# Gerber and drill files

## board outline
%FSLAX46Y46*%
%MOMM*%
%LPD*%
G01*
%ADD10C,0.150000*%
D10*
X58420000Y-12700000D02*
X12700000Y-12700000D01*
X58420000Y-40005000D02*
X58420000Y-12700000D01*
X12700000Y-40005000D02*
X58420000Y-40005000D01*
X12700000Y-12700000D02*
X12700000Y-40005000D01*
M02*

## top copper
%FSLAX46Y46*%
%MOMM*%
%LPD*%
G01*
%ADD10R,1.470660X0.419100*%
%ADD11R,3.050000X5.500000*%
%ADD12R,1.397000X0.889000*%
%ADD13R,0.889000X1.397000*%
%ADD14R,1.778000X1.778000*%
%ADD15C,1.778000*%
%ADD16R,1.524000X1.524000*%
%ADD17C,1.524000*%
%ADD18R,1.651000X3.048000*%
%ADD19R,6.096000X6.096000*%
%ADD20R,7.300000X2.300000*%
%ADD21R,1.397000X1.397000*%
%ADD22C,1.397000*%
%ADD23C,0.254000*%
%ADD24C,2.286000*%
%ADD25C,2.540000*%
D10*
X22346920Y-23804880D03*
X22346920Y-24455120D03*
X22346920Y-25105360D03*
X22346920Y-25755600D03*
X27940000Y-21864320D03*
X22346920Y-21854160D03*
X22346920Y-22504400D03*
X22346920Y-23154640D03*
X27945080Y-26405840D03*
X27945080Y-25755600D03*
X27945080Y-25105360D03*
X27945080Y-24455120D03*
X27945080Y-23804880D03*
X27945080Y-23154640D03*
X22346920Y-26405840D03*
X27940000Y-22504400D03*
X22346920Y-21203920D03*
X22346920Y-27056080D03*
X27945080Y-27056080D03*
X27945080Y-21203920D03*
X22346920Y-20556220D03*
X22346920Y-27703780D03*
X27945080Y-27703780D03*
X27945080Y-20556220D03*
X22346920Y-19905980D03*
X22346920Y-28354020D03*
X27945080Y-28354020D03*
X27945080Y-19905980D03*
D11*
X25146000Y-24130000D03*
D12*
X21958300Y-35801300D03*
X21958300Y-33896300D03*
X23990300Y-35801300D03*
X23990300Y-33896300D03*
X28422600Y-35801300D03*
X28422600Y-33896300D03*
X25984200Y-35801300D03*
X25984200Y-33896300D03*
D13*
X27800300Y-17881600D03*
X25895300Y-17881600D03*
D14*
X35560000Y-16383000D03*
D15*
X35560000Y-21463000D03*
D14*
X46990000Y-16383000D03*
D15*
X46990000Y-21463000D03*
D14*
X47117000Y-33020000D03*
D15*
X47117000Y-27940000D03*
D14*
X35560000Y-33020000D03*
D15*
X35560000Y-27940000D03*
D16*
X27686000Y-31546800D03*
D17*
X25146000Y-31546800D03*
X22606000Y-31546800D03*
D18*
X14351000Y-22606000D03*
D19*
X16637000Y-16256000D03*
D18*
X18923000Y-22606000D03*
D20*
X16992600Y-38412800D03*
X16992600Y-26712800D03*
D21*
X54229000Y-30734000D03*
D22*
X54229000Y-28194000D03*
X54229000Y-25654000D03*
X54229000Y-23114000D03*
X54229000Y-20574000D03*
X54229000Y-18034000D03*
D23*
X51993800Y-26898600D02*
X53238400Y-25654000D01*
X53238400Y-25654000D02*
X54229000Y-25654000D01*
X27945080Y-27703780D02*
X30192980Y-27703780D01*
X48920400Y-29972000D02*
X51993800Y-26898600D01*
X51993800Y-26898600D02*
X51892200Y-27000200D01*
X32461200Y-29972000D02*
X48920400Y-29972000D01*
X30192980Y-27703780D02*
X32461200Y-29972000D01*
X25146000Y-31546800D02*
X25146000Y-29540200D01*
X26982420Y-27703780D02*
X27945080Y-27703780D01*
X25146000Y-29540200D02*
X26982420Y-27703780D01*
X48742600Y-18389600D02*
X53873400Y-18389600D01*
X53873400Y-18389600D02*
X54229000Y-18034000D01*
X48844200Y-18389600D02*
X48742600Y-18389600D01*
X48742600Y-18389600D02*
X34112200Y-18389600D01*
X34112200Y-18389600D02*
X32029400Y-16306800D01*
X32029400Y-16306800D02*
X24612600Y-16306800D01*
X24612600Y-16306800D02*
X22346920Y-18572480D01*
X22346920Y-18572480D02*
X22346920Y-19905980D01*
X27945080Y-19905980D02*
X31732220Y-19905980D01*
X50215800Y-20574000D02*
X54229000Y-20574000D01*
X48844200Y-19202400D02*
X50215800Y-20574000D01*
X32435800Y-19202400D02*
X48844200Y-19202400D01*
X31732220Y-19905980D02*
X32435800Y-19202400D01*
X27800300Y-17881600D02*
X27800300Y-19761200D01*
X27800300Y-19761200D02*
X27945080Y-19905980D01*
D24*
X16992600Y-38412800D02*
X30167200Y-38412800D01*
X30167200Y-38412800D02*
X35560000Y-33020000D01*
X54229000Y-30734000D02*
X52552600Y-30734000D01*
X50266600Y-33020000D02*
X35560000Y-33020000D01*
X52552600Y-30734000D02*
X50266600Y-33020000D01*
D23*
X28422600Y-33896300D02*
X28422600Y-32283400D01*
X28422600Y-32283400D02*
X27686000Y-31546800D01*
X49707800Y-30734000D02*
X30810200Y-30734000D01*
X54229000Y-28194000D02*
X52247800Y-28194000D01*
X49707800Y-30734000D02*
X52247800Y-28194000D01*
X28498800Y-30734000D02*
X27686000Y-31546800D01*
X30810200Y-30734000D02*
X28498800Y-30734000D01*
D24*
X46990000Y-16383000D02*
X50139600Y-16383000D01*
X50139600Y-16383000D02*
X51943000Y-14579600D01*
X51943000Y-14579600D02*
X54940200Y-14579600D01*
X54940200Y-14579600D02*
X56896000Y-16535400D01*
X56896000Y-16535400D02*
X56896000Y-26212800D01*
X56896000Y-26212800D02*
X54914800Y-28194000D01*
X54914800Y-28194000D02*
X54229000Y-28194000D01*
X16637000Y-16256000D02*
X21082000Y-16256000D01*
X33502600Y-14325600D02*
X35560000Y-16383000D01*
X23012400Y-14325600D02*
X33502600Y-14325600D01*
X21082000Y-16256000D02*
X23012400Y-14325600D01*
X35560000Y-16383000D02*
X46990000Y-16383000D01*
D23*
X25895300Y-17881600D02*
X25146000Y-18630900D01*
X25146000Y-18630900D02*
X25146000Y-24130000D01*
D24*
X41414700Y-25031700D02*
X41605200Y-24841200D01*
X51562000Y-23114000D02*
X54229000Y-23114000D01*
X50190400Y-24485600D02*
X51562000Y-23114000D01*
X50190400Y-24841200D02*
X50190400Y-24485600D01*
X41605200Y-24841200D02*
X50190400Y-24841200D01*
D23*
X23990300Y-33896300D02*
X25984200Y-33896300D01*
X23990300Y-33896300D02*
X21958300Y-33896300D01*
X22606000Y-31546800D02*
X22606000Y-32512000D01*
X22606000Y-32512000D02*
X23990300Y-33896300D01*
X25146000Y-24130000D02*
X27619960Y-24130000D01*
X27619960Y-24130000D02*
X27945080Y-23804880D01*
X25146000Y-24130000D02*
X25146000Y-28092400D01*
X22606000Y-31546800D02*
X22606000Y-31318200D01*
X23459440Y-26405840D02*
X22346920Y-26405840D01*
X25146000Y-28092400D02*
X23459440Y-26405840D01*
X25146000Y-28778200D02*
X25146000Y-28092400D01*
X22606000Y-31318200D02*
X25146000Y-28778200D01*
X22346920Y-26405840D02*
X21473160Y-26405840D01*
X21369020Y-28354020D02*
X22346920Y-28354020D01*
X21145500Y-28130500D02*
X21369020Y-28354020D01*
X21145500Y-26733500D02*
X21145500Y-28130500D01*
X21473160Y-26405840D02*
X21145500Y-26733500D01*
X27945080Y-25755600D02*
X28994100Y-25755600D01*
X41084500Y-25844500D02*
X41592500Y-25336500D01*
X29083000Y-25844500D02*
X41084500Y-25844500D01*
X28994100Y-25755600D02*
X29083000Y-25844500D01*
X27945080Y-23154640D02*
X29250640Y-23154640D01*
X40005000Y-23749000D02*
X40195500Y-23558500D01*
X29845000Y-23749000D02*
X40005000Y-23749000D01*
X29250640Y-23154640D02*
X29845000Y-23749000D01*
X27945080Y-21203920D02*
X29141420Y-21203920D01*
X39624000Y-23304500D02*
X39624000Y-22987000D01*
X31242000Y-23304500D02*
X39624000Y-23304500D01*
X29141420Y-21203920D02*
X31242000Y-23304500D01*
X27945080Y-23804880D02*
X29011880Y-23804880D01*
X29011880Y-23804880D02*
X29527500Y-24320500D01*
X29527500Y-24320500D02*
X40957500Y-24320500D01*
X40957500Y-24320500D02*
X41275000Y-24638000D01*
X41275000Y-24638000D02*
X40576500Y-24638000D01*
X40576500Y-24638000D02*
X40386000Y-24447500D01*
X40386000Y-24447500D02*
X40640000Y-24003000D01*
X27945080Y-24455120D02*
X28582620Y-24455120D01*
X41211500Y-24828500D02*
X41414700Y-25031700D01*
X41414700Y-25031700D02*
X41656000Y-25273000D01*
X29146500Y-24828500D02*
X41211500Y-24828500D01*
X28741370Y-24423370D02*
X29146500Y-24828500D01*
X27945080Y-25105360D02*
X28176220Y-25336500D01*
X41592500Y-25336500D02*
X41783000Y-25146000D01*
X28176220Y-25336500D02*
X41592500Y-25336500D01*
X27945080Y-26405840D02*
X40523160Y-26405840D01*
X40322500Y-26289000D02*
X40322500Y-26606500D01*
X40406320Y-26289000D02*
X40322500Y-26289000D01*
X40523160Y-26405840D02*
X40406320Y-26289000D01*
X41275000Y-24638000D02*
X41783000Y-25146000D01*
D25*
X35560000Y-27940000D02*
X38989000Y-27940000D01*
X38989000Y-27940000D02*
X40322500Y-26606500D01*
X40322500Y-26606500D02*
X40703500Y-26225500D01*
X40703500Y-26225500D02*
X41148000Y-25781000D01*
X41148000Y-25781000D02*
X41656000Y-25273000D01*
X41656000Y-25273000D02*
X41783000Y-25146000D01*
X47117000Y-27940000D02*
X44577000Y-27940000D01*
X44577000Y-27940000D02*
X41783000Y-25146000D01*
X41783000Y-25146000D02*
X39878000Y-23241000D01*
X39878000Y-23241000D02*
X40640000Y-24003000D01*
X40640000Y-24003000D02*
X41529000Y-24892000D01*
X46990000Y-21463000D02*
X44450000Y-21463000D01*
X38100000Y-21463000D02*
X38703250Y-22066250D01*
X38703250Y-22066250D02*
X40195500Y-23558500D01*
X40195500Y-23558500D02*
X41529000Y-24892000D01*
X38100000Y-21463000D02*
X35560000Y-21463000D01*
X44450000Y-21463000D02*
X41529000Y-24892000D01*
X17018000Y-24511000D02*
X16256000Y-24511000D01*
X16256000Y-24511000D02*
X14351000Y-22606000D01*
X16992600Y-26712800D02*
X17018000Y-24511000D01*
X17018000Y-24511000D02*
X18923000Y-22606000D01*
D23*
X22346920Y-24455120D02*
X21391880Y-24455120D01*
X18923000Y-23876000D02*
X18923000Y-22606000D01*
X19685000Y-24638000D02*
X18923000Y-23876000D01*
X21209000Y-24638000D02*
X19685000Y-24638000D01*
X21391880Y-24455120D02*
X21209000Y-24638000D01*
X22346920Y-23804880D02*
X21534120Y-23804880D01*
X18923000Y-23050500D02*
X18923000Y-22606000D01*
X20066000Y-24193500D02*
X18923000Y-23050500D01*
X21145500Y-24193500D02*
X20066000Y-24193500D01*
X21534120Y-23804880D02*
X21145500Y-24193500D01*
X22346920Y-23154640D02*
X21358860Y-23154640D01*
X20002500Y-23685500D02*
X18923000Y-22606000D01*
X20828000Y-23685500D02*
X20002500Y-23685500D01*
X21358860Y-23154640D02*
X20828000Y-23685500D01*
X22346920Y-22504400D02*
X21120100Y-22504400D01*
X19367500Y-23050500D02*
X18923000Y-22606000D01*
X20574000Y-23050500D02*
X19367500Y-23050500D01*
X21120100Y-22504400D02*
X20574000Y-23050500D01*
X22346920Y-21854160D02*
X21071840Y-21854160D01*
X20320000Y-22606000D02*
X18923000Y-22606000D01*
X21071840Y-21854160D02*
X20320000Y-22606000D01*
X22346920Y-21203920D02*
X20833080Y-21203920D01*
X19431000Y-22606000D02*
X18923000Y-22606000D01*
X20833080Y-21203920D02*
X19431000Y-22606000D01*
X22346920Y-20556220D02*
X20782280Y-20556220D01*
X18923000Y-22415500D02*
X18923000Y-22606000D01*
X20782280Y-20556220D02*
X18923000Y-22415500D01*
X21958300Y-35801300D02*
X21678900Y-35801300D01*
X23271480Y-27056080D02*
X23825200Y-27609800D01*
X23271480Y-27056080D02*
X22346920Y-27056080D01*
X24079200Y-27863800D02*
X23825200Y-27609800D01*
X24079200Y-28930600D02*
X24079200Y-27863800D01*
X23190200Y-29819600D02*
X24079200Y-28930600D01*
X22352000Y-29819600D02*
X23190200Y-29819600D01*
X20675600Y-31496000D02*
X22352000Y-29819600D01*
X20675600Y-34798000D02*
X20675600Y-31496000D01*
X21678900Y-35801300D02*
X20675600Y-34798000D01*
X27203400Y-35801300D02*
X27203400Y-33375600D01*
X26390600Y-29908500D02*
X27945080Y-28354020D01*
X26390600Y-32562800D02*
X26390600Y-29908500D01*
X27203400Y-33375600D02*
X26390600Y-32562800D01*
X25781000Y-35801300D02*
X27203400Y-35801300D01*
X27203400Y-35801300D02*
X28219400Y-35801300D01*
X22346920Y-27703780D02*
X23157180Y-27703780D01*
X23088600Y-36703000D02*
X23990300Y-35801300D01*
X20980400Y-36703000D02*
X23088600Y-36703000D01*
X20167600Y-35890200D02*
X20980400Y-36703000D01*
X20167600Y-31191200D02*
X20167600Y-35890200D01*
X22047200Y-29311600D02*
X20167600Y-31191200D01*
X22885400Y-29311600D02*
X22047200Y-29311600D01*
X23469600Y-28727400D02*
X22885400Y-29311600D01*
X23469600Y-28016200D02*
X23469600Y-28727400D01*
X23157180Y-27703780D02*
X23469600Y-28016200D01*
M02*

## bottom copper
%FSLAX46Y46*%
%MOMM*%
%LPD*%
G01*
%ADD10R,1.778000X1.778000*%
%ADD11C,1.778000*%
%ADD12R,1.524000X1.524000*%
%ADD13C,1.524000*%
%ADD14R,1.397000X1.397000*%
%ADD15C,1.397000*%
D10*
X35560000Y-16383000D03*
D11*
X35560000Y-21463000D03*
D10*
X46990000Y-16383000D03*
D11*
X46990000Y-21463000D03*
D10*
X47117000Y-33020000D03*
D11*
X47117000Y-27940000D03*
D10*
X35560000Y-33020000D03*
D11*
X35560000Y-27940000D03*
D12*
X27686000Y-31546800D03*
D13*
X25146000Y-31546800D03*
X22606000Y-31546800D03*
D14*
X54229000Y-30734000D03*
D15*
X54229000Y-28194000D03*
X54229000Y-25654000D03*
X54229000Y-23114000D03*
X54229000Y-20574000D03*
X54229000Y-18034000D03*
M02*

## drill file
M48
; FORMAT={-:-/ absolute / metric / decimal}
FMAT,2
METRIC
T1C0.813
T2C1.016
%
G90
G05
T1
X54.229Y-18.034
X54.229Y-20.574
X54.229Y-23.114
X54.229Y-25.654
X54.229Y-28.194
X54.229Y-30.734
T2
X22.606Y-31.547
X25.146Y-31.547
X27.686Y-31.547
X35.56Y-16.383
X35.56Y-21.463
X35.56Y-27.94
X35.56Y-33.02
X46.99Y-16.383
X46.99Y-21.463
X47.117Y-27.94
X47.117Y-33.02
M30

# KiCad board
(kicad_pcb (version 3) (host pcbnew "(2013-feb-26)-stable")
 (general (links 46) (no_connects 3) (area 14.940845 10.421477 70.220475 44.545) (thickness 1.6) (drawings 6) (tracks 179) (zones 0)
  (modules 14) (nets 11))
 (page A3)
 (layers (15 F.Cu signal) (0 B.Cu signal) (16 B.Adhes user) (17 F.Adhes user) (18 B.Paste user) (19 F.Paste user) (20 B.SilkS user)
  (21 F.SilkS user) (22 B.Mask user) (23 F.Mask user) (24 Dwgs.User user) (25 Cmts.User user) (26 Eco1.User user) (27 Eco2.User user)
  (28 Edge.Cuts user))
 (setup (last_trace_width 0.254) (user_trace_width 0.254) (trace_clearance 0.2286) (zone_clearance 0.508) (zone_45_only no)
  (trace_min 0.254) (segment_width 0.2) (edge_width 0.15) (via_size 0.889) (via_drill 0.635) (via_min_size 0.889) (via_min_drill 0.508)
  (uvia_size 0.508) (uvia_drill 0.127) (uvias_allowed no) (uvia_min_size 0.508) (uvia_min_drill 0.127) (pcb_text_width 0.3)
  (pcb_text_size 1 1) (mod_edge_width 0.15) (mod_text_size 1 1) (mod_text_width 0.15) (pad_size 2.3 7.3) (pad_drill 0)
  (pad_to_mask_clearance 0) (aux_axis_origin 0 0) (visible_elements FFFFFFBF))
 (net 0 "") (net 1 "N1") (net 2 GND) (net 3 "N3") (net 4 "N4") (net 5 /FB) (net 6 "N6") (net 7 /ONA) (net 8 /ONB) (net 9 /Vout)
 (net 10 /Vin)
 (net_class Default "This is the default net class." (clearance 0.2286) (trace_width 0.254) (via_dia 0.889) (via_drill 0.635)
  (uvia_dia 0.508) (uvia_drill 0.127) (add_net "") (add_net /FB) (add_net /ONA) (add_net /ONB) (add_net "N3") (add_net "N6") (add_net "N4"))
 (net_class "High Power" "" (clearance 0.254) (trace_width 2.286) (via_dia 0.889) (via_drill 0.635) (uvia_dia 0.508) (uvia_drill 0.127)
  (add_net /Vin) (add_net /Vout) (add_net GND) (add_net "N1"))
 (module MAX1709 (layer F.Cu) (at 25.146 24.13 270) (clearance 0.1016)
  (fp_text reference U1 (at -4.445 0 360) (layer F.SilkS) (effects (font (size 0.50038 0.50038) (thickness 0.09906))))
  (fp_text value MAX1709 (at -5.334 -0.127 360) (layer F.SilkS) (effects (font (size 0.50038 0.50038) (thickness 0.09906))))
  (pad 2 smd rect (at -0.32512 2.79908 270) (size 0.4191 1.47066) (layers F.Cu F.Paste F.Mask) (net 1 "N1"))
  (pad 2 smd rect (at 0.32512 2.79908 270) (size 0.4191 1.47066) (layers F.Cu F.Paste F.Mask) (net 1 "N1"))
  (pad 9 smd rect (at 0.97536 2.79908 270) (size 0.4191 1.47066) (layers F.Cu F.Paste F.Mask))
  (pad 10 smd rect (at 1.6256 2.79908 270) (size 0.4191 1.47066) (layers F.Cu F.Paste F.Mask))
  (pad 25 smd rect (at -2.26568 -2.794 270) (size 0.4191 1.47066) (layers F.Cu F.Paste F.Mask))
  (pad 2 smd rect (at -2.27584 2.79908 270) (size 0.4191 1.47066) (layers F.Cu F.Paste F.Mask) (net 1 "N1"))
  (pad 2 smd rect (at -1.6256 2.79908 270) (size 0.4191 1.47066) (layers F.Cu F.Paste F.Mask) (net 1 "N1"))
  (pad 2 smd rect (at -0.97536 2.79908 270) (size 0.4191 1.47066) (layers F.Cu F.Paste F.Mask) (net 1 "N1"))
  (pad 18 smd rect (at 2.27584 -2.79908 270) (size 0.4191 1.47066) (layers F.Cu F.Paste F.Mask) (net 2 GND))
  (pad 18 smd rect (at 1.6256 -2.79908 270) (size 0.4191 1.47066) (layers F.Cu F.Paste F.Mask) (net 2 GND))
  (pad 18 smd rect (at 0.97536 -2.79908 270) (size 0.4191 1.47066) (layers F.Cu F.Paste F.Mask) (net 2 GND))
  (pad 18 smd rect (at 0.32512 -2.79908 270) (size 0.4191 1.47066) (layers F.Cu F.Paste F.Mask) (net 2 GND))
  (pad 18 smd rect (at -0.32512 -2.79908 270) (size 0.4191 1.47066) (layers F.Cu F.Paste F.Mask) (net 2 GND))
  (pad 18 smd rect (at -0.97536 -2.79908 270) (size 0.4191 1.47066) (layers F.Cu F.Paste F.Mask) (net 2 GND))
  (pad 11 smd rect (at 2.27584 2.79908 270) (size 0.4191 1.47066) (layers F.Cu F.Paste F.Mask) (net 2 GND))
  (pad 24 smd rect (at -1.6256 -2.794 270) (size 0.4191 1.47066) (layers F.Cu F.Paste F.Mask))
  (pad 2 smd rect (at -2.92608 2.79908 270) (size 0.4191 1.47066) (layers F.Cu F.Paste F.Mask) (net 1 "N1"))
  (pad 12 smd rect (at 2.92608 2.79908 270) (size 0.4191 1.47066) (layers F.Cu F.Paste F.Mask) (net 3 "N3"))
  (pad 17 smd rect (at 2.92608 -2.79908 270) (size 0.4191 1.47066) (layers F.Cu F.Paste F.Mask))
  (pad 26 smd rect (at -2.92608 -2.79908 270) (size 0.4191 1.47066) (layers F.Cu F.Paste F.Mask) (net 2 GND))
  (pad 2 smd rect (at -3.57378 2.79908 270) (size 0.4191 1.47066) (layers F.Cu F.Paste F.Mask) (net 1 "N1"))
  (pad 13 smd rect (at 3.57378 2.79908 270) (size 0.4191 1.47066) (layers F.Cu F.Paste F.Mask) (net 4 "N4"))
  (pad 16 smd rect (at 3.57378 -2.79908 270) (size 0.4191 1.47066) (layers F.Cu F.Paste F.Mask) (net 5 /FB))
  (pad 27 smd rect (at -3.57378 -2.79908 270) (size 0.4191 1.47066) (layers F.Cu F.Paste F.Mask) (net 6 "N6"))
  (pad 1 smd rect (at -4.22402 2.79908 270) (size 0.4191 1.47066) (layers F.Cu F.Paste F.Mask) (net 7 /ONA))
  (pad 11 smd rect (at 4.22402 2.79908 270) (size 0.4191 1.47066) (layers F.Cu F.Paste F.Mask) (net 2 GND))
  (pad 15 smd rect (at 4.22402 -2.79908 270) (size 0.4191 1.47066) (layers F.Cu F.Paste F.Mask) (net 6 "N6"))
  (pad 28 smd rect (at -4.22402 -2.79908 270) (size 0.4191 1.47066) (layers F.Cu F.Paste F.Mask) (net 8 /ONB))
  (pad 18 smd rect (at 0 0 270) (size 5.5 3.05) (layers F.Cu F.Paste F.Mask) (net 2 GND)))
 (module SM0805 (layer F.Cu) (at 21.9583 34.8488 90)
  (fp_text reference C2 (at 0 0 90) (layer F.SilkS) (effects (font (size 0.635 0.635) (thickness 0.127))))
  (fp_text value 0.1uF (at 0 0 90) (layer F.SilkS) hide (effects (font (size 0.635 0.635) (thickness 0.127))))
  (pad 1 smd rect (at -0.9525 0 90) (size 0.889 1.397) (layers F.Cu F.Paste F.Mask) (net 3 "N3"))
  (pad 2 smd rect (at 0.9525 0 90) (size 0.889 1.397) (layers F.Cu F.Paste F.Mask) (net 2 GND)))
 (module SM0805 (layer F.Cu) (at 23.9903 34.8488 90)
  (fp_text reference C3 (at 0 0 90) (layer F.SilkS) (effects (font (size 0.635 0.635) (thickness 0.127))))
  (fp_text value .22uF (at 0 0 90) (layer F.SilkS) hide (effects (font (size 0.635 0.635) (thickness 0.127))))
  (pad 1 smd rect (at -0.9525 0 90) (size 0.889 1.397) (layers F.Cu F.Paste F.Mask) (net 4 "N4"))
  (pad 2 smd rect (at 0.9525 0 90) (size 0.889 1.397) (layers F.Cu F.Paste F.Mask) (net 2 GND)))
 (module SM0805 (layer F.Cu) (at 28.4226 34.8488 90)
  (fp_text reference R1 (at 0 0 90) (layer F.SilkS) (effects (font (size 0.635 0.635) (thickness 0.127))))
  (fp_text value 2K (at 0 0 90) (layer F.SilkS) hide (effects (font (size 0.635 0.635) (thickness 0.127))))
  (pad 1 smd rect (at -0.9525 0 90) (size 0.889 1.397) (layers F.Cu F.Paste F.Mask) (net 6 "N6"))
  (pad 2 smd rect (at 0.9525 0 90) (size 0.889 1.397) (layers F.Cu F.Paste F.Mask) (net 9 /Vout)))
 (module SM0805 (layer F.Cu) (at 25.9842 34.8488 90)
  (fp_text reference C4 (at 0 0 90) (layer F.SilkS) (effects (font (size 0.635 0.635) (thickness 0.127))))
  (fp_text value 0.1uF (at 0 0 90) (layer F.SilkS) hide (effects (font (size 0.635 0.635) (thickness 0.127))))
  (pad 1 smd rect (at -0.9525 0 90) (size 0.889 1.397) (layers F.Cu F.Paste F.Mask) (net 6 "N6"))
  (pad 2 smd rect (at 0.9525 0 90) (size 0.889 1.397) (layers F.Cu F.Paste F.Mask) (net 2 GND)))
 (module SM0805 (layer F.Cu) (at 26.8478 17.8816 180)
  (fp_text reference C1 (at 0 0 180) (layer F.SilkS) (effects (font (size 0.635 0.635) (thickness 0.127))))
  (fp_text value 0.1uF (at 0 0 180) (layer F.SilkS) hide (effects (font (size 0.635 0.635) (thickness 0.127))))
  (pad 1 smd rect (at -0.9525 0 180) (size 0.889 1.397) (layers F.Cu F.Paste F.Mask) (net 8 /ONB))
  (pad 2 smd rect (at 0.9525 0 180) (size 0.889 1.397) (layers F.Cu F.Paste F.Mask) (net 2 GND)))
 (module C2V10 (layer B.Cu) (at 35.56 18.923 270)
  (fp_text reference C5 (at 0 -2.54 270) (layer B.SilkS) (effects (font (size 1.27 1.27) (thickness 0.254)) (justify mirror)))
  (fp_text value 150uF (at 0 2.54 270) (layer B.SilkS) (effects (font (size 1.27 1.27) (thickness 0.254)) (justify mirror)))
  (pad 1 thru_hole rect (at -2.54 0 270) (size 1.778 1.778) (drill 1.016) (layers *.Cu *.Mask B.SilkS) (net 9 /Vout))
  (pad 2 thru_hole circle (at 2.54 0 270) (size 1.778 1.778) (drill 1.016) (layers *.Cu *.Mask B.SilkS) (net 2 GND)))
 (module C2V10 (layer B.Cu) (at 46.99 18.923 270)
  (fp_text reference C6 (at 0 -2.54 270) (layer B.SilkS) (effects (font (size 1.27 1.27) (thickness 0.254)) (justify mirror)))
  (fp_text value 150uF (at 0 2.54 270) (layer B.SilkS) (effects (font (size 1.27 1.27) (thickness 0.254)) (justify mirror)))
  (pad 1 thru_hole rect (at -2.54 0 270) (size 1.778 1.778) (drill 1.016) (layers *.Cu *.Mask B.SilkS) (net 9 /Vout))
  (pad 2 thru_hole circle (at 2.54 0 270) (size 1.778 1.778) (drill 1.016) (layers *.Cu *.Mask B.SilkS) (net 2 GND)))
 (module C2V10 (layer B.Cu) (at 47.117 30.48 90)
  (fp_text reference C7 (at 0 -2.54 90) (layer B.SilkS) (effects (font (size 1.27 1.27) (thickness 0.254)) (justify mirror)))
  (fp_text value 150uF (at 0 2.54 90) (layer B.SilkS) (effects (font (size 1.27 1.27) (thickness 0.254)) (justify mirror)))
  (pad 1 thru_hole rect (at -2.54 0 90) (size 1.778 1.778) (drill 1.016) (layers *.Cu *.Mask B.SilkS) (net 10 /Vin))
  (pad 2 thru_hole circle (at 2.54 0 90) (size 1.778 1.778) (drill 1.016) (layers *.Cu *.Mask B.SilkS) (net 2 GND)))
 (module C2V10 (layer B.Cu) (at 35.56 30.48 90)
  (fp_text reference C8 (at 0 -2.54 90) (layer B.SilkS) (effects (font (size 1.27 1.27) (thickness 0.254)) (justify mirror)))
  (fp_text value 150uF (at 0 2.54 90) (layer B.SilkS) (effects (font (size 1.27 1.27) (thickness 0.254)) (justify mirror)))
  (pad 1 thru_hole rect (at -2.54 0 90) (size 1.778 1.778) (drill 1.016) (layers *.Cu *.Mask B.SilkS) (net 10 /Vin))
  (pad 2 thru_hole circle (at 2.54 0 90) (size 1.778 1.778) (drill 1.016) (layers *.Cu *.Mask B.SilkS) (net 2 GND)))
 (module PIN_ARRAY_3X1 (layer F.Cu) (at 25.146 31.5468 180)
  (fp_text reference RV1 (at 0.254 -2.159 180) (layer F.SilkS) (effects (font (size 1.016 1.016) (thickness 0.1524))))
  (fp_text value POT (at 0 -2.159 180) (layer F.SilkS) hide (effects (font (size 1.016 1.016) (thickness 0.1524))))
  (pad 1 thru_hole rect (at -2.54 0 180) (size 1.524 1.524) (drill 1.016) (layers *.Cu *.Mask F.SilkS) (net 9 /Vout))
  (pad 2 thru_hole circle (at 0 0 180) (size 1.524 1.524) (drill 1.016) (layers *.Cu *.Mask F.SilkS) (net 5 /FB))
  (pad 3 thru_hole circle (at 2.54 0 180) (size 1.524 1.524) (drill 1.016) (layers *.Cu *.Mask F.SilkS) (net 2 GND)))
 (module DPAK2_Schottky (layer F.Cu) (at 16.637 22.606)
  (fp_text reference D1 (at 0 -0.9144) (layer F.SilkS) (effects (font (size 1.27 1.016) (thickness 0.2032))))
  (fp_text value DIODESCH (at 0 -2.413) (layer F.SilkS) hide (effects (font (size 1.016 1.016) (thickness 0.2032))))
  (pad 1 smd rect (at -2.286 0) (size 1.651 3.048) (layers F.Cu F.Paste F.Mask) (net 1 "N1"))
  (pad 2 smd rect (at 0 -6.35) (size 6.096 6.096) (layers F.Cu F.Paste F.Mask) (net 9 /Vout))
  (pad 1 smd rect (at 2.286 0) (size 1.651 3.048) (layers F.Cu F.Paste F.Mask) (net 1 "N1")))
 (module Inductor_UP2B (layer F.Cu) (at 16.9926 32.5628 90)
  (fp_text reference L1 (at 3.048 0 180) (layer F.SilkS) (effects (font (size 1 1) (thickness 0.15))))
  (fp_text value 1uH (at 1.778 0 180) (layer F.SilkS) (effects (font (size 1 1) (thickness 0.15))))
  (pad 1 smd rect (at -5.85 0 90) (size 2.3 7.3) (layers F.Cu F.Paste F.Mask) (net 10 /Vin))
  (pad 2 smd rect (at 5.85 0 90) (size 2.3 7.3) (layers F.Cu F.Paste F.Mask) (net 1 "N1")))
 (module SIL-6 (layer F.Cu) (at 54.229 24.384 90)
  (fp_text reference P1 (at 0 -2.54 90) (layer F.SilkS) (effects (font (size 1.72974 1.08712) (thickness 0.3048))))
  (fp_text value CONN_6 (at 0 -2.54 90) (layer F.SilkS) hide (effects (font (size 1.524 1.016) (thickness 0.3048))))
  (pad 1 thru_hole rect (at -6.35 0 90) (size 1.397 1.397) (drill 0.8128) (layers *.Cu *.Mask F.SilkS) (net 10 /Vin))
  (pad 2 thru_hole circle (at -3.81 0 90) (size 1.397 1.397) (drill 0.8128) (layers *.Cu *.Mask F.SilkS) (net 9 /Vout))
  (pad 3 thru_hole circle (at -1.27 0 90) (size 1.397 1.397) (drill 0.8128) (layers *.Cu *.Mask F.SilkS) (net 5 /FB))
  (pad 4 thru_hole circle (at 1.27 0 90) (size 1.397 1.397) (drill 0.8128) (layers *.Cu *.Mask F.SilkS) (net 2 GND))
  (pad 5 thru_hole circle (at 3.81 0 90) (size 1.397 1.397) (drill 0.8128) (layers *.Cu *.Mask F.SilkS) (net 8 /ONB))
  (pad 6 thru_hole circle (at 6.35 0 90) (size 1.397 1.397) (drill 0.8128) (layers *.Cu *.Mask F.SilkS) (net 7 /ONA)))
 (gr_line (start 58.42 12.7) (end 12.7 12.7) (angle 90) (layer Edge.Cuts) (width 0.15))
 (gr_line (start 58.42 40.005) (end 58.42 12.7) (angle 90) (layer Edge.Cuts) (width 0.15))
 (gr_line (start 12.7 40.005) (end 58.42 40.005) (angle 90) (layer Edge.Cuts) (width 0.15))
 (gr_line (start 12.7 12.7) (end 12.7 40.005) (angle 90) (layer Edge.Cuts) (width 0.15))
 (segment (start 51.9938 26.8986) (end 53.2384 25.654) (width 0.254) (layer F.Cu) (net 5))
 (segment (start 53.2384 25.654) (end 54.229 25.654) (width 0.254) (layer F.Cu) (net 5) (status 20))
 (segment (start 27.94508 27.70378) (end 30.19298 27.70378) (width 0.254) (layer F.Cu) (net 5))
 (segment (start 48.9204 29.972) (end 51.9938 26.8986) (width 0.254) (layer F.Cu) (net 5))
 (segment (start 51.9938 26.8986) (end 51.8922 27.0002) (width 0.254) (layer F.Cu) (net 5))
 (segment (start 32.4612 29.972) (end 48.9204 29.972) (width 0.254) (layer F.Cu) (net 5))
 (segment (start 30.19298 27.70378) (end 32.4612 29.972) (width 0.254) (layer F.Cu) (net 5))
 (segment (start 25.146 31.5468) (end 25.146 29.5402) (width 0.254) (layer F.Cu) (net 5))
 (segment (start 26.98242 27.70378) (end 27.94508 27.70378) (width 0.254) (layer F.Cu) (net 5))
 (segment (start 25.146 29.5402) (end 26.98242 27.70378) (width 0.254) (layer F.Cu) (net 5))
 (segment (start 48.7426 18.3896) (end 53.8734 18.3896) (width 0.254) (layer F.Cu) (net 7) (status 20))
 (segment (start 53.8734 18.3896) (end 54.229 18.034) (width 0.254) (layer F.Cu) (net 7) (status 30))
 (segment (start 48.8442 18.3896) (end 48.7426 18.3896) (width 0.254) (layer F.Cu) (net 7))
 (segment (start 48.7426 18.3896) (end 34.1122 18.3896) (width 0.254) (layer F.Cu) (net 7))
 (segment (start 34.1122 18.3896) (end 32.0294 16.3068) (width 0.254) (layer F.Cu) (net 7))
 (segment (start 32.0294 16.3068) (end 24.6126 16.3068) (width 0.254) (layer F.Cu) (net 7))
 (segment (start 24.6126 16.3068) (end 22.34692 18.57248) (width 0.254) (layer F.Cu) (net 7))
 (segment (start 22.34692 18.57248) (end 22.34692 19.90598) (width 0.254) (layer F.Cu) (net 7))
 (segment (start 27.94508 19.90598) (end 31.73222 19.90598) (width 0.254) (layer F.Cu) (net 8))
 (segment (start 50.2158 20.574) (end 54.229 20.574) (width 0.254) (layer F.Cu) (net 8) (status 20))
 (segment (start 48.8442 19.2024) (end 50.2158 20.574) (width 0.254) (layer F.Cu) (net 8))
 (segment (start 32.4358 19.2024) (end 48.8442 19.2024) (width 0.254) (layer F.Cu) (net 8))
 (segment (start 31.73222 19.90598) (end 32.4358 19.2024) (width 0.254) (layer F.Cu) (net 8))
 (segment (start 27.8003 17.8816) (end 27.8003 19.7612) (width 0.254) (layer F.Cu) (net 8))
 (segment (start 27.8003 19.7612) (end 27.94508 19.90598) (width 0.254) (layer F.Cu) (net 8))
 (segment (start 16.9926 38.4128) (end 30.1672 38.4128) (width 2.286) (layer F.Cu) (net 10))
 (segment (start 30.1672 38.4128) (end 35.56 33.02) (width 2.286) (layer F.Cu) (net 10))
 (segment (start 54.229 30.734) (end 52.5526 30.734) (width 2.286) (layer F.Cu) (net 10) (status 10))
 (segment (start 50.2666 33.02) (end 35.56 33.02) (width 2.286) (layer F.Cu) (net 10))
 (segment (start 52.5526 30.734) (end 50.2666 33.02) (width 2.286) (layer F.Cu) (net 10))
 (segment (start 28.4226 33.8963) (end 28.4226 32.2834) (width 0.254) (layer F.Cu) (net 9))
 (segment (start 28.4226 32.2834) (end 27.686 31.5468) (width 0.254) (layer F.Cu) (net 9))
 (segment (start 49.7078 30.734) (end 30.8102 30.734) (width 0.254) (layer F.Cu) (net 9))
 (segment (start 54.229 28.194) (end 52.2478 28.194) (width 0.254) (layer F.Cu) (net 9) (status 10))
 (segment (start 49.7078 30.734) (end 52.2478 28.194) (width 0.254) (layer F.Cu) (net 9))
 (segment (start 28.4988 30.734) (end 27.686 31.5468) (width 0.254) (layer F.Cu) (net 9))
 (segment (start 30.8102 30.734) (end 28.4988 30.734) (width 0.254) (layer F.Cu) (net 9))
 (segment (start 46.99 16.383) (end 50.1396 16.383) (width 2.286) (layer F.Cu) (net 9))
 (segment (start 50.1396 16.383) (end 51.943 14.5796) (width 2.286) (layer F.Cu) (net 9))
 (segment (start 51.943 14.5796) (end 54.9402 14.5796) (width 2.286) (layer F.Cu) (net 9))
 (segment (start 54.9402 14.5796) (end 56.896 16.5354) (width 2.286) (layer F.Cu) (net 9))
 (segment (start 56.896 16.5354) (end 56.896 26.2128) (width 2.286) (layer F.Cu) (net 9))
 (segment (start 56.896 26.2128) (end 54.9148 28.194) (width 2.286) (layer F.Cu) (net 9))
 (segment (start 54.9148 28.194) (end 54.229 28.194) (width 2.286) (layer F.Cu) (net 9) (status 20))
 (segment (start 16.637 16.256) (end 21.082 16.256) (width 2.286) (layer F.Cu) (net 9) (status 10))
 (segment (start 33.5026 14.3256) (end 35.56 16.383) (width 2.286) (layer F.Cu) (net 9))
 (segment (start 23.0124 14.3256) (end 33.5026 14.3256) (width 2.286) (layer F.Cu) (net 9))
 (segment (start 21.082 16.256) (end 23.0124 14.3256) (width 2.286) (layer F.Cu) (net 9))
 (segment (start 35.56 16.383) (end 46.99 16.383) (width 2.286) (layer F.Cu) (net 9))
 (segment (start 25.8953 17.8816) (end 25.146 18.6309) (width 0.254) (layer F.Cu) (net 2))
 (segment (start 25.146 18.6309) (end 25.146 24.13) (width 0.254) (layer F.Cu) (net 2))
 (segment (start 41.4147 25.0317) (end 41.6052 24.8412) (width 2.286) (layer F.Cu) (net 2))
 (segment (start 51.562 23.114) (end 54.229 23.114) (width 2.286) (layer F.Cu) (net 2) (status 20))
 (segment (start 50.1904 24.4856) (end 51.562 23.114) (width 2.286) (layer F.Cu) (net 2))
 (segment (start 50.1904 24.8412) (end 50.1904 24.4856) (width 2.286) (layer F.Cu) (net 2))
 (segment (start 41.6052 24.8412) (end 50.1904 24.8412) (width 2.286) (layer F.Cu) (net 2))
 (segment (start 23.9903 33.8963) (end 25.9842 33.8963) (width 0.254) (layer F.Cu) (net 2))
 (segment (start 23.9903 33.8963) (end 21.9583 33.8963) (width 0.254) (layer F.Cu) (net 2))
 (segment (start 22.606 31.5468) (end 22.606 32.512) (width 0.254) (layer F.Cu) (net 2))
 (segment (start 22.606 32.512) (end 23.9903 33.8963) (width 0.254) (layer F.Cu) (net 2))
 (segment (start 25.146 24.13) (end 27.61996 24.13) (width 0.254) (layer F.Cu) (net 2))
 (segment (start 27.61996 24.13) (end 27.94508 23.80488) (width 0.254) (layer F.Cu) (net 2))
 (segment (start 25.146 24.13) (end 25.146 28.0924) (width 0.254) (layer F.Cu) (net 2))
 (segment (start 22.606 31.5468) (end 22.606 31.3182) (width 0.254) (layer F.Cu) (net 2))
 (segment (start 23.45944 26.40584) (end 22.34692 26.40584) (width 0.254) (layer F.Cu) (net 2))
 (segment (start 25.146 28.0924) (end 23.45944 26.40584) (width 0.254) (layer F.Cu) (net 2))
 (segment (start 25.146 28.7782) (end 25.146 28.0924) (width 0.254) (layer F.Cu) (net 2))
 (segment (start 22.606 31.3182) (end 25.146 28.7782) (width 0.254) (layer F.Cu) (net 2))
 (segment (start 22.34692 26.40584) (end 21.47316 26.40584) (width 0.254) (layer F.Cu) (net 2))
 (segment (start 21.36902 28.35402) (end 22.34692 28.35402) (width 0.254) (layer F.Cu) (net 2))
 (segment (start 21.1455 28.1305) (end 21.36902 28.35402) (width 0.254) (layer F.Cu) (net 2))
 (segment (start 21.1455 26.7335) (end 21.1455 28.1305) (width 0.254) (layer F.Cu) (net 2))
 (segment (start 21.47316 26.40584) (end 21.1455 26.7335) (width 0.254) (layer F.Cu) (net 2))
 (segment (start 27.94508 25.7556) (end 28.9941 25.7556) (width 0.254) (layer F.Cu) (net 2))
 (segment (start 41.0845 25.8445) (end 41.5925 25.3365) (width 0.254) (layer F.Cu) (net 2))
 (segment (start 29.083 25.8445) (end 41.0845 25.8445) (width 0.254) (layer F.Cu) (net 2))
 (segment (start 28.9941 25.7556) (end 29.083 25.8445) (width 0.254) (layer F.Cu) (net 2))
 (segment (start 27.94508 23.15464) (end 29.25064 23.15464) (width 0.254) (layer F.Cu) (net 2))
 (segment (start 40.005 23.749) (end 40.1955 23.5585) (width 0.254) (layer F.Cu) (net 2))
 (segment (start 29.845 23.749) (end 40.005 23.749) (width 0.254) (layer F.Cu) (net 2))
 (segment (start 29.25064 23.15464) (end 29.845 23.749) (width 0.254) (layer F.Cu) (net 2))
 (segment (start 27.94508 21.20392) (end 29.14142 21.20392) (width 0.254) (layer F.Cu) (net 2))
 (segment (start 39.624 23.3045) (end 39.624 22.987) (width 0.254) (layer F.Cu) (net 2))
 (segment (start 31.242 23.3045) (end 39.624 23.3045) (width 0.254) (layer F.Cu) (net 2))
 (segment (start 29.14142 21.20392) (end 31.242 23.3045) (width 0.254) (layer F.Cu) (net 2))
 (segment (start 27.94508 23.80488) (end 29.01188 23.80488) (width 0.254) (layer F.Cu) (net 2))
 (segment (start 29.01188 23.80488) (end 29.5275 24.3205) (width 0.254) (layer F.Cu) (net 2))
 (segment (start 29.5275 24.3205) (end 40.9575 24.3205) (width 0.254) (layer F.Cu) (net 2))
 (segment (start 40.9575 24.3205) (end 41.275 24.638) (width 0.254) (layer F.Cu) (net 2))
 (segment (start 41.275 24.638) (end 40.5765 24.638) (width 0.254) (layer F.Cu) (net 2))
 (segment (start 40.5765 24.638) (end 40.386 24.4475) (width 0.254) (layer F.Cu) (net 2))
 (segment (start 40.386 24.4475) (end 40.64 24.003) (width 0.254) (layer F.Cu) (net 2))
 (segment (start 27.94508 24.45512) (end 28.58262 24.45512) (width 0.254) (layer F.Cu) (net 2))
 (segment (start 41.2115 24.8285) (end 41.4147 25.0317) (width 0.254) (layer F.Cu) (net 2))
 (segment (start 41.4147 25.0317) (end 41.656 25.273) (width 0.254) (layer F.Cu) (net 2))
 (segment (start 29.1465 24.8285) (end 41.2115 24.8285) (width 0.254) (layer F.Cu) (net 2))
 (segment (start 28.74137 24.42337) (end 29.1465 24.8285) (width 0.254) (layer F.Cu) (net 2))
 (segment (start 27.94508 25.10536) (end 28.17622 25.3365) (width 0.254) (layer F.Cu) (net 2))
 (segment (start 41.5925 25.3365) (end 41.783 25.146) (width 0.254) (layer F.Cu) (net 2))
 (segment (start 28.17622 25.3365) (end 41.5925 25.3365) (width 0.254) (layer F.Cu) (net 2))
 (segment (start 27.94508 26.40584) (end 40.52316 26.40584) (width 0.254) (layer F.Cu) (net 2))
 (segment (start 40.3225 26.289) (end 40.3225 26.6065) (width 0.254) (layer F.Cu) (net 2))
 (segment (start 40.40632 26.289) (end 40.3225 26.289) (width 0.254) (layer F.Cu) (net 2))
 (segment (start 40.52316 26.40584) (end 40.40632 26.289) (width 0.254) (layer F.Cu) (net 2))
 (segment (start 41.275 24.638) (end 41.783 25.146) (width 0.254) (layer F.Cu) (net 2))
 (segment (start 35.56 27.94) (end 38.989 27.94) (width 2.54) (layer F.Cu) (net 2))
 (segment (start 38.989 27.94) (end 40.3225 26.6065) (width 2.54) (layer F.Cu) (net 2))
 (segment (start 40.3225 26.6065) (end 40.7035 26.2255) (width 2.54) (layer F.Cu) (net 2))
 (segment (start 40.7035 26.2255) (end 41.148 25.781) (width 2.54) (layer F.Cu) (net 2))
 (segment (start 41.148 25.781) (end 41.656 25.273) (width 2.54) (layer F.Cu) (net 2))
 (segment (start 41.656 25.273) (end 41.783 25.146) (width 2.54) (layer F.Cu) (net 2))
 (segment (start 47.117 27.94) (end 44.577 27.94) (width 2.54) (layer F.Cu) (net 2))
 (segment (start 44.577 27.94) (end 41.783 25.146) (width 2.54) (layer F.Cu) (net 2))
 (segment (start 41.783 25.146) (end 39.878 23.241) (width 2.54) (layer F.Cu) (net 2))
 (segment (start 39.878 23.241) (end 40.64 24.003) (width 2.54) (layer F.Cu) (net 2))
 (segment (start 40.64 24.003) (end 41.529 24.892) (width 2.54) (layer F.Cu) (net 2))
 (segment (start 46.99 21.463) (end 44.45 21.463) (width 2.54) (layer F.Cu) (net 2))
 (segment (start 38.1 21.463) (end 38.70325 22.06625) (width 2.54) (layer F.Cu) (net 2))
 (segment (start 38.70325 22.06625) (end 40.1955 23.5585) (width 2.54) (layer F.Cu) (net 2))
 (segment (start 40.1955 23.5585) (end 41.529 24.892) (width 2.54) (layer F.Cu) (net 2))
 (segment (start 38.1 21.463) (end 35.56 21.463) (width 2.54) (layer F.Cu) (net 2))
 (segment (start 44.45 21.463) (end 41.529 24.892) (width 2.54) (layer F.Cu) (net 2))
 (segment (start 17.018 24.511) (end 16.256 24.511) (width 2.54) (layer F.Cu) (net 1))
 (segment (start 16.256 24.511) (end 14.351 22.606) (width 2.54) (layer F.Cu) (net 1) (status 20))
 (segment (start 16.9926 26.7128) (end 17.018 24.511) (width 2.54) (layer F.Cu) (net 1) (status 10))
 (segment (start 17.018 24.511) (end 18.923 22.606) (width 2.54) (layer F.Cu) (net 1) (status 20))
 (segment (start 22.34692 24.45512) (end 21.39188 24.45512) (width 0.254) (layer F.Cu) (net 1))
 (segment (start 18.923 23.876) (end 18.923 22.606) (width 0.254) (layer F.Cu) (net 1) (status 30))
 (segment (start 19.685 24.638) (end 18.923 23.876) (width 0.254) (layer F.Cu) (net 1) (status 20))
 (segment (start 21.209 24.638) (end 19.685 24.638) (width 0.254) (layer F.Cu) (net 1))
 (segment (start 21.39188 24.45512) (end 21.209 24.638) (width 0.254) (layer F.Cu) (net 1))
 (segment (start 22.34692 23.80488) (end 21.53412 23.80488) (width 0.254) (layer F.Cu) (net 1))
 (segment (start 18.923 23.0505) (end 18.923 22.606) (width 0.254) (layer F.Cu) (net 1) (status 30))
 (segment (start 20.066 24.1935) (end 18.923 23.0505) (width 0.254) (layer F.Cu) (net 1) (status 20))
 (segment (start 21.1455 24.1935) (end 20.066 24.1935) (width 0.254) (layer F.Cu) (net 1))
 (segment (start 21.53412 23.80488) (end 21.1455 24.1935) (width 0.254) (layer F.Cu) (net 1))
 (segment (start 22.34692 23.15464) (end 21.35886 23.15464) (width 0.254) (layer F.Cu) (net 1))
 (segment (start 20.0025 23.6855) (end 18.923 22.606) (width 0.254) (layer F.Cu) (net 1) (status 20))
 (segment (start 20.828 23.6855) (end 20.0025 23.6855) (width 0.254) (layer F.Cu) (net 1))
 (segment (start 21.35886 23.15464) (end 20.828 23.6855) (width 0.254) (layer F.Cu) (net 1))
 (segment (start 22.34692 22.5044) (end 21.1201 22.5044) (width 0.254) (layer F.Cu) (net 1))
 (segment (start 19.3675 23.0505) (end 18.923 22.606) (width 0.254) (layer F.Cu) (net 1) (status 30))
 (segment (start 20.574 23.0505) (end 19.3675 23.0505) (width 0.254) (layer F.Cu) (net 1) (status 20))
 (segment (start 21.1201 22.5044) (end 20.574 23.0505) (width 0.254) (layer F.Cu) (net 1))
 (segment (start 22.34692 21.85416) (end 21.07184 21.85416) (width 0.254) (layer F.Cu) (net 1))
 (segment (start 20.32 22.606) (end 18.923 22.606) (width 0.254) (layer F.Cu) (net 1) (status 20))
 (segment (start 21.07184 21.85416) (end 20.32 22.606) (width 0.254) (layer F.Cu) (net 1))
 (segment (start 22.34692 21.20392) (end 20.83308 21.20392) (width 0.254) (layer F.Cu) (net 1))
 (segment (start 19.431 22.606) (end 18.923 22.606) (width 0.254) (layer F.Cu) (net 1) (status 30))
 (segment (start 20.83308 21.20392) (end 19.431 22.606) (width 0.254) (layer F.Cu) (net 1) (status 20))
 (segment (start 22.34692 20.55622) (end 20.78228 20.55622) (width 0.254) (layer F.Cu) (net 1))
 (segment (start 18.923 22.4155) (end 18.923 22.606) (width 0.254) (layer F.Cu) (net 1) (status 30))
 (segment (start 20.78228 20.55622) (end 18.923 22.4155) (width 0.254) (layer F.Cu) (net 1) (status 20))
 (segment (start 21.9583 35.8013) (end 21.6789 35.8013) (width 0.254) (layer F.Cu) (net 3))
 (segment (start 23.27148 27.05608) (end 23.8252 27.6098) (width 0.254) (layer F.Cu) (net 3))
 (segment (start 23.27148 27.05608) (end 22.34692 27.05608) (width 0.254) (layer F.Cu) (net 3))
 (segment (start 24.0792 27.8638) (end 23.8252 27.6098) (width 0.254) (layer F.Cu) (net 3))
 (segment (start 24.0792 28.9306) (end 24.0792 27.8638) (width 0.254) (layer F.Cu) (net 3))
 (segment (start 23.1902 29.8196) (end 24.0792 28.9306) (width 0.254) (layer F.Cu) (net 3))
 (segment (start 22.352 29.8196) (end 23.1902 29.8196) (width 0.254) (layer F.Cu) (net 3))
 (segment (start 20.6756 31.496) (end 22.352 29.8196) (width 0.254) (layer F.Cu) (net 3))
 (segment (start 20.6756 34.798) (end 20.6756 31.496) (width 0.254) (layer F.Cu) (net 3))
 (segment (start 21.6789 35.8013) (end 20.6756 34.798) (width 0.254) (layer F.Cu) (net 3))
 (segment (start 27.2034 35.8013) (end 27.2034 33.3756) (width 0.254) (layer F.Cu) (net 6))
 (segment (start 26.3906 29.9085) (end 27.94508 28.35402) (width 0.254) (layer F.Cu) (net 6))
 (segment (start 26.3906 32.5628) (end 26.3906 29.9085) (width 0.254) (layer F.Cu) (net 6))
 (segment (start 27.2034 33.3756) (end 26.3906 32.5628) (width 0.254) (layer F.Cu) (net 6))
 (segment (start 25.781 35.8013) (end 27.2034 35.8013) (width 0.254) (layer F.Cu) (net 6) (status 20))
 (segment (start 27.2034 35.8013) (end 28.2194 35.8013) (width 0.254) (layer F.Cu) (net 6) (status 20))
 (segment (start 22.34692 27.70378) (end 23.15718 27.70378) (width 0.254) (layer F.Cu) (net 4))
 (segment (start 23.0886 36.703) (end 23.9903 35.8013) (width 0.254) (layer F.Cu) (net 4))
 (segment (start 20.9804 36.703) (end 23.0886 36.703) (width 0.254) (layer F.Cu) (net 4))
 (segment (start 20.1676 35.8902) (end 20.9804 36.703) (width 0.254) (layer F.Cu) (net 4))
 (segment (start 20.1676 31.1912) (end 20.1676 35.8902) (width 0.254) (layer F.Cu) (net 4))
 (segment (start 22.0472 29.3116) (end 20.1676 31.1912) (width 0.254) (layer F.Cu) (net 4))
 (segment (start 22.8854 29.3116) (end 22.0472 29.3116) (width 0.254) (layer F.Cu) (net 4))
 (segment (start 23.4696 28.7274) (end 22.8854 29.3116) (width 0.254) (layer F.Cu) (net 4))
 (segment (start 23.4696 28.0162) (end 23.4696 28.7274) (width 0.254) (layer F.Cu) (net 4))
 (segment (start 23.15718 27.70378) (end 23.4696 28.0162) (width 0.254) (layer F.Cu) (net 4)))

